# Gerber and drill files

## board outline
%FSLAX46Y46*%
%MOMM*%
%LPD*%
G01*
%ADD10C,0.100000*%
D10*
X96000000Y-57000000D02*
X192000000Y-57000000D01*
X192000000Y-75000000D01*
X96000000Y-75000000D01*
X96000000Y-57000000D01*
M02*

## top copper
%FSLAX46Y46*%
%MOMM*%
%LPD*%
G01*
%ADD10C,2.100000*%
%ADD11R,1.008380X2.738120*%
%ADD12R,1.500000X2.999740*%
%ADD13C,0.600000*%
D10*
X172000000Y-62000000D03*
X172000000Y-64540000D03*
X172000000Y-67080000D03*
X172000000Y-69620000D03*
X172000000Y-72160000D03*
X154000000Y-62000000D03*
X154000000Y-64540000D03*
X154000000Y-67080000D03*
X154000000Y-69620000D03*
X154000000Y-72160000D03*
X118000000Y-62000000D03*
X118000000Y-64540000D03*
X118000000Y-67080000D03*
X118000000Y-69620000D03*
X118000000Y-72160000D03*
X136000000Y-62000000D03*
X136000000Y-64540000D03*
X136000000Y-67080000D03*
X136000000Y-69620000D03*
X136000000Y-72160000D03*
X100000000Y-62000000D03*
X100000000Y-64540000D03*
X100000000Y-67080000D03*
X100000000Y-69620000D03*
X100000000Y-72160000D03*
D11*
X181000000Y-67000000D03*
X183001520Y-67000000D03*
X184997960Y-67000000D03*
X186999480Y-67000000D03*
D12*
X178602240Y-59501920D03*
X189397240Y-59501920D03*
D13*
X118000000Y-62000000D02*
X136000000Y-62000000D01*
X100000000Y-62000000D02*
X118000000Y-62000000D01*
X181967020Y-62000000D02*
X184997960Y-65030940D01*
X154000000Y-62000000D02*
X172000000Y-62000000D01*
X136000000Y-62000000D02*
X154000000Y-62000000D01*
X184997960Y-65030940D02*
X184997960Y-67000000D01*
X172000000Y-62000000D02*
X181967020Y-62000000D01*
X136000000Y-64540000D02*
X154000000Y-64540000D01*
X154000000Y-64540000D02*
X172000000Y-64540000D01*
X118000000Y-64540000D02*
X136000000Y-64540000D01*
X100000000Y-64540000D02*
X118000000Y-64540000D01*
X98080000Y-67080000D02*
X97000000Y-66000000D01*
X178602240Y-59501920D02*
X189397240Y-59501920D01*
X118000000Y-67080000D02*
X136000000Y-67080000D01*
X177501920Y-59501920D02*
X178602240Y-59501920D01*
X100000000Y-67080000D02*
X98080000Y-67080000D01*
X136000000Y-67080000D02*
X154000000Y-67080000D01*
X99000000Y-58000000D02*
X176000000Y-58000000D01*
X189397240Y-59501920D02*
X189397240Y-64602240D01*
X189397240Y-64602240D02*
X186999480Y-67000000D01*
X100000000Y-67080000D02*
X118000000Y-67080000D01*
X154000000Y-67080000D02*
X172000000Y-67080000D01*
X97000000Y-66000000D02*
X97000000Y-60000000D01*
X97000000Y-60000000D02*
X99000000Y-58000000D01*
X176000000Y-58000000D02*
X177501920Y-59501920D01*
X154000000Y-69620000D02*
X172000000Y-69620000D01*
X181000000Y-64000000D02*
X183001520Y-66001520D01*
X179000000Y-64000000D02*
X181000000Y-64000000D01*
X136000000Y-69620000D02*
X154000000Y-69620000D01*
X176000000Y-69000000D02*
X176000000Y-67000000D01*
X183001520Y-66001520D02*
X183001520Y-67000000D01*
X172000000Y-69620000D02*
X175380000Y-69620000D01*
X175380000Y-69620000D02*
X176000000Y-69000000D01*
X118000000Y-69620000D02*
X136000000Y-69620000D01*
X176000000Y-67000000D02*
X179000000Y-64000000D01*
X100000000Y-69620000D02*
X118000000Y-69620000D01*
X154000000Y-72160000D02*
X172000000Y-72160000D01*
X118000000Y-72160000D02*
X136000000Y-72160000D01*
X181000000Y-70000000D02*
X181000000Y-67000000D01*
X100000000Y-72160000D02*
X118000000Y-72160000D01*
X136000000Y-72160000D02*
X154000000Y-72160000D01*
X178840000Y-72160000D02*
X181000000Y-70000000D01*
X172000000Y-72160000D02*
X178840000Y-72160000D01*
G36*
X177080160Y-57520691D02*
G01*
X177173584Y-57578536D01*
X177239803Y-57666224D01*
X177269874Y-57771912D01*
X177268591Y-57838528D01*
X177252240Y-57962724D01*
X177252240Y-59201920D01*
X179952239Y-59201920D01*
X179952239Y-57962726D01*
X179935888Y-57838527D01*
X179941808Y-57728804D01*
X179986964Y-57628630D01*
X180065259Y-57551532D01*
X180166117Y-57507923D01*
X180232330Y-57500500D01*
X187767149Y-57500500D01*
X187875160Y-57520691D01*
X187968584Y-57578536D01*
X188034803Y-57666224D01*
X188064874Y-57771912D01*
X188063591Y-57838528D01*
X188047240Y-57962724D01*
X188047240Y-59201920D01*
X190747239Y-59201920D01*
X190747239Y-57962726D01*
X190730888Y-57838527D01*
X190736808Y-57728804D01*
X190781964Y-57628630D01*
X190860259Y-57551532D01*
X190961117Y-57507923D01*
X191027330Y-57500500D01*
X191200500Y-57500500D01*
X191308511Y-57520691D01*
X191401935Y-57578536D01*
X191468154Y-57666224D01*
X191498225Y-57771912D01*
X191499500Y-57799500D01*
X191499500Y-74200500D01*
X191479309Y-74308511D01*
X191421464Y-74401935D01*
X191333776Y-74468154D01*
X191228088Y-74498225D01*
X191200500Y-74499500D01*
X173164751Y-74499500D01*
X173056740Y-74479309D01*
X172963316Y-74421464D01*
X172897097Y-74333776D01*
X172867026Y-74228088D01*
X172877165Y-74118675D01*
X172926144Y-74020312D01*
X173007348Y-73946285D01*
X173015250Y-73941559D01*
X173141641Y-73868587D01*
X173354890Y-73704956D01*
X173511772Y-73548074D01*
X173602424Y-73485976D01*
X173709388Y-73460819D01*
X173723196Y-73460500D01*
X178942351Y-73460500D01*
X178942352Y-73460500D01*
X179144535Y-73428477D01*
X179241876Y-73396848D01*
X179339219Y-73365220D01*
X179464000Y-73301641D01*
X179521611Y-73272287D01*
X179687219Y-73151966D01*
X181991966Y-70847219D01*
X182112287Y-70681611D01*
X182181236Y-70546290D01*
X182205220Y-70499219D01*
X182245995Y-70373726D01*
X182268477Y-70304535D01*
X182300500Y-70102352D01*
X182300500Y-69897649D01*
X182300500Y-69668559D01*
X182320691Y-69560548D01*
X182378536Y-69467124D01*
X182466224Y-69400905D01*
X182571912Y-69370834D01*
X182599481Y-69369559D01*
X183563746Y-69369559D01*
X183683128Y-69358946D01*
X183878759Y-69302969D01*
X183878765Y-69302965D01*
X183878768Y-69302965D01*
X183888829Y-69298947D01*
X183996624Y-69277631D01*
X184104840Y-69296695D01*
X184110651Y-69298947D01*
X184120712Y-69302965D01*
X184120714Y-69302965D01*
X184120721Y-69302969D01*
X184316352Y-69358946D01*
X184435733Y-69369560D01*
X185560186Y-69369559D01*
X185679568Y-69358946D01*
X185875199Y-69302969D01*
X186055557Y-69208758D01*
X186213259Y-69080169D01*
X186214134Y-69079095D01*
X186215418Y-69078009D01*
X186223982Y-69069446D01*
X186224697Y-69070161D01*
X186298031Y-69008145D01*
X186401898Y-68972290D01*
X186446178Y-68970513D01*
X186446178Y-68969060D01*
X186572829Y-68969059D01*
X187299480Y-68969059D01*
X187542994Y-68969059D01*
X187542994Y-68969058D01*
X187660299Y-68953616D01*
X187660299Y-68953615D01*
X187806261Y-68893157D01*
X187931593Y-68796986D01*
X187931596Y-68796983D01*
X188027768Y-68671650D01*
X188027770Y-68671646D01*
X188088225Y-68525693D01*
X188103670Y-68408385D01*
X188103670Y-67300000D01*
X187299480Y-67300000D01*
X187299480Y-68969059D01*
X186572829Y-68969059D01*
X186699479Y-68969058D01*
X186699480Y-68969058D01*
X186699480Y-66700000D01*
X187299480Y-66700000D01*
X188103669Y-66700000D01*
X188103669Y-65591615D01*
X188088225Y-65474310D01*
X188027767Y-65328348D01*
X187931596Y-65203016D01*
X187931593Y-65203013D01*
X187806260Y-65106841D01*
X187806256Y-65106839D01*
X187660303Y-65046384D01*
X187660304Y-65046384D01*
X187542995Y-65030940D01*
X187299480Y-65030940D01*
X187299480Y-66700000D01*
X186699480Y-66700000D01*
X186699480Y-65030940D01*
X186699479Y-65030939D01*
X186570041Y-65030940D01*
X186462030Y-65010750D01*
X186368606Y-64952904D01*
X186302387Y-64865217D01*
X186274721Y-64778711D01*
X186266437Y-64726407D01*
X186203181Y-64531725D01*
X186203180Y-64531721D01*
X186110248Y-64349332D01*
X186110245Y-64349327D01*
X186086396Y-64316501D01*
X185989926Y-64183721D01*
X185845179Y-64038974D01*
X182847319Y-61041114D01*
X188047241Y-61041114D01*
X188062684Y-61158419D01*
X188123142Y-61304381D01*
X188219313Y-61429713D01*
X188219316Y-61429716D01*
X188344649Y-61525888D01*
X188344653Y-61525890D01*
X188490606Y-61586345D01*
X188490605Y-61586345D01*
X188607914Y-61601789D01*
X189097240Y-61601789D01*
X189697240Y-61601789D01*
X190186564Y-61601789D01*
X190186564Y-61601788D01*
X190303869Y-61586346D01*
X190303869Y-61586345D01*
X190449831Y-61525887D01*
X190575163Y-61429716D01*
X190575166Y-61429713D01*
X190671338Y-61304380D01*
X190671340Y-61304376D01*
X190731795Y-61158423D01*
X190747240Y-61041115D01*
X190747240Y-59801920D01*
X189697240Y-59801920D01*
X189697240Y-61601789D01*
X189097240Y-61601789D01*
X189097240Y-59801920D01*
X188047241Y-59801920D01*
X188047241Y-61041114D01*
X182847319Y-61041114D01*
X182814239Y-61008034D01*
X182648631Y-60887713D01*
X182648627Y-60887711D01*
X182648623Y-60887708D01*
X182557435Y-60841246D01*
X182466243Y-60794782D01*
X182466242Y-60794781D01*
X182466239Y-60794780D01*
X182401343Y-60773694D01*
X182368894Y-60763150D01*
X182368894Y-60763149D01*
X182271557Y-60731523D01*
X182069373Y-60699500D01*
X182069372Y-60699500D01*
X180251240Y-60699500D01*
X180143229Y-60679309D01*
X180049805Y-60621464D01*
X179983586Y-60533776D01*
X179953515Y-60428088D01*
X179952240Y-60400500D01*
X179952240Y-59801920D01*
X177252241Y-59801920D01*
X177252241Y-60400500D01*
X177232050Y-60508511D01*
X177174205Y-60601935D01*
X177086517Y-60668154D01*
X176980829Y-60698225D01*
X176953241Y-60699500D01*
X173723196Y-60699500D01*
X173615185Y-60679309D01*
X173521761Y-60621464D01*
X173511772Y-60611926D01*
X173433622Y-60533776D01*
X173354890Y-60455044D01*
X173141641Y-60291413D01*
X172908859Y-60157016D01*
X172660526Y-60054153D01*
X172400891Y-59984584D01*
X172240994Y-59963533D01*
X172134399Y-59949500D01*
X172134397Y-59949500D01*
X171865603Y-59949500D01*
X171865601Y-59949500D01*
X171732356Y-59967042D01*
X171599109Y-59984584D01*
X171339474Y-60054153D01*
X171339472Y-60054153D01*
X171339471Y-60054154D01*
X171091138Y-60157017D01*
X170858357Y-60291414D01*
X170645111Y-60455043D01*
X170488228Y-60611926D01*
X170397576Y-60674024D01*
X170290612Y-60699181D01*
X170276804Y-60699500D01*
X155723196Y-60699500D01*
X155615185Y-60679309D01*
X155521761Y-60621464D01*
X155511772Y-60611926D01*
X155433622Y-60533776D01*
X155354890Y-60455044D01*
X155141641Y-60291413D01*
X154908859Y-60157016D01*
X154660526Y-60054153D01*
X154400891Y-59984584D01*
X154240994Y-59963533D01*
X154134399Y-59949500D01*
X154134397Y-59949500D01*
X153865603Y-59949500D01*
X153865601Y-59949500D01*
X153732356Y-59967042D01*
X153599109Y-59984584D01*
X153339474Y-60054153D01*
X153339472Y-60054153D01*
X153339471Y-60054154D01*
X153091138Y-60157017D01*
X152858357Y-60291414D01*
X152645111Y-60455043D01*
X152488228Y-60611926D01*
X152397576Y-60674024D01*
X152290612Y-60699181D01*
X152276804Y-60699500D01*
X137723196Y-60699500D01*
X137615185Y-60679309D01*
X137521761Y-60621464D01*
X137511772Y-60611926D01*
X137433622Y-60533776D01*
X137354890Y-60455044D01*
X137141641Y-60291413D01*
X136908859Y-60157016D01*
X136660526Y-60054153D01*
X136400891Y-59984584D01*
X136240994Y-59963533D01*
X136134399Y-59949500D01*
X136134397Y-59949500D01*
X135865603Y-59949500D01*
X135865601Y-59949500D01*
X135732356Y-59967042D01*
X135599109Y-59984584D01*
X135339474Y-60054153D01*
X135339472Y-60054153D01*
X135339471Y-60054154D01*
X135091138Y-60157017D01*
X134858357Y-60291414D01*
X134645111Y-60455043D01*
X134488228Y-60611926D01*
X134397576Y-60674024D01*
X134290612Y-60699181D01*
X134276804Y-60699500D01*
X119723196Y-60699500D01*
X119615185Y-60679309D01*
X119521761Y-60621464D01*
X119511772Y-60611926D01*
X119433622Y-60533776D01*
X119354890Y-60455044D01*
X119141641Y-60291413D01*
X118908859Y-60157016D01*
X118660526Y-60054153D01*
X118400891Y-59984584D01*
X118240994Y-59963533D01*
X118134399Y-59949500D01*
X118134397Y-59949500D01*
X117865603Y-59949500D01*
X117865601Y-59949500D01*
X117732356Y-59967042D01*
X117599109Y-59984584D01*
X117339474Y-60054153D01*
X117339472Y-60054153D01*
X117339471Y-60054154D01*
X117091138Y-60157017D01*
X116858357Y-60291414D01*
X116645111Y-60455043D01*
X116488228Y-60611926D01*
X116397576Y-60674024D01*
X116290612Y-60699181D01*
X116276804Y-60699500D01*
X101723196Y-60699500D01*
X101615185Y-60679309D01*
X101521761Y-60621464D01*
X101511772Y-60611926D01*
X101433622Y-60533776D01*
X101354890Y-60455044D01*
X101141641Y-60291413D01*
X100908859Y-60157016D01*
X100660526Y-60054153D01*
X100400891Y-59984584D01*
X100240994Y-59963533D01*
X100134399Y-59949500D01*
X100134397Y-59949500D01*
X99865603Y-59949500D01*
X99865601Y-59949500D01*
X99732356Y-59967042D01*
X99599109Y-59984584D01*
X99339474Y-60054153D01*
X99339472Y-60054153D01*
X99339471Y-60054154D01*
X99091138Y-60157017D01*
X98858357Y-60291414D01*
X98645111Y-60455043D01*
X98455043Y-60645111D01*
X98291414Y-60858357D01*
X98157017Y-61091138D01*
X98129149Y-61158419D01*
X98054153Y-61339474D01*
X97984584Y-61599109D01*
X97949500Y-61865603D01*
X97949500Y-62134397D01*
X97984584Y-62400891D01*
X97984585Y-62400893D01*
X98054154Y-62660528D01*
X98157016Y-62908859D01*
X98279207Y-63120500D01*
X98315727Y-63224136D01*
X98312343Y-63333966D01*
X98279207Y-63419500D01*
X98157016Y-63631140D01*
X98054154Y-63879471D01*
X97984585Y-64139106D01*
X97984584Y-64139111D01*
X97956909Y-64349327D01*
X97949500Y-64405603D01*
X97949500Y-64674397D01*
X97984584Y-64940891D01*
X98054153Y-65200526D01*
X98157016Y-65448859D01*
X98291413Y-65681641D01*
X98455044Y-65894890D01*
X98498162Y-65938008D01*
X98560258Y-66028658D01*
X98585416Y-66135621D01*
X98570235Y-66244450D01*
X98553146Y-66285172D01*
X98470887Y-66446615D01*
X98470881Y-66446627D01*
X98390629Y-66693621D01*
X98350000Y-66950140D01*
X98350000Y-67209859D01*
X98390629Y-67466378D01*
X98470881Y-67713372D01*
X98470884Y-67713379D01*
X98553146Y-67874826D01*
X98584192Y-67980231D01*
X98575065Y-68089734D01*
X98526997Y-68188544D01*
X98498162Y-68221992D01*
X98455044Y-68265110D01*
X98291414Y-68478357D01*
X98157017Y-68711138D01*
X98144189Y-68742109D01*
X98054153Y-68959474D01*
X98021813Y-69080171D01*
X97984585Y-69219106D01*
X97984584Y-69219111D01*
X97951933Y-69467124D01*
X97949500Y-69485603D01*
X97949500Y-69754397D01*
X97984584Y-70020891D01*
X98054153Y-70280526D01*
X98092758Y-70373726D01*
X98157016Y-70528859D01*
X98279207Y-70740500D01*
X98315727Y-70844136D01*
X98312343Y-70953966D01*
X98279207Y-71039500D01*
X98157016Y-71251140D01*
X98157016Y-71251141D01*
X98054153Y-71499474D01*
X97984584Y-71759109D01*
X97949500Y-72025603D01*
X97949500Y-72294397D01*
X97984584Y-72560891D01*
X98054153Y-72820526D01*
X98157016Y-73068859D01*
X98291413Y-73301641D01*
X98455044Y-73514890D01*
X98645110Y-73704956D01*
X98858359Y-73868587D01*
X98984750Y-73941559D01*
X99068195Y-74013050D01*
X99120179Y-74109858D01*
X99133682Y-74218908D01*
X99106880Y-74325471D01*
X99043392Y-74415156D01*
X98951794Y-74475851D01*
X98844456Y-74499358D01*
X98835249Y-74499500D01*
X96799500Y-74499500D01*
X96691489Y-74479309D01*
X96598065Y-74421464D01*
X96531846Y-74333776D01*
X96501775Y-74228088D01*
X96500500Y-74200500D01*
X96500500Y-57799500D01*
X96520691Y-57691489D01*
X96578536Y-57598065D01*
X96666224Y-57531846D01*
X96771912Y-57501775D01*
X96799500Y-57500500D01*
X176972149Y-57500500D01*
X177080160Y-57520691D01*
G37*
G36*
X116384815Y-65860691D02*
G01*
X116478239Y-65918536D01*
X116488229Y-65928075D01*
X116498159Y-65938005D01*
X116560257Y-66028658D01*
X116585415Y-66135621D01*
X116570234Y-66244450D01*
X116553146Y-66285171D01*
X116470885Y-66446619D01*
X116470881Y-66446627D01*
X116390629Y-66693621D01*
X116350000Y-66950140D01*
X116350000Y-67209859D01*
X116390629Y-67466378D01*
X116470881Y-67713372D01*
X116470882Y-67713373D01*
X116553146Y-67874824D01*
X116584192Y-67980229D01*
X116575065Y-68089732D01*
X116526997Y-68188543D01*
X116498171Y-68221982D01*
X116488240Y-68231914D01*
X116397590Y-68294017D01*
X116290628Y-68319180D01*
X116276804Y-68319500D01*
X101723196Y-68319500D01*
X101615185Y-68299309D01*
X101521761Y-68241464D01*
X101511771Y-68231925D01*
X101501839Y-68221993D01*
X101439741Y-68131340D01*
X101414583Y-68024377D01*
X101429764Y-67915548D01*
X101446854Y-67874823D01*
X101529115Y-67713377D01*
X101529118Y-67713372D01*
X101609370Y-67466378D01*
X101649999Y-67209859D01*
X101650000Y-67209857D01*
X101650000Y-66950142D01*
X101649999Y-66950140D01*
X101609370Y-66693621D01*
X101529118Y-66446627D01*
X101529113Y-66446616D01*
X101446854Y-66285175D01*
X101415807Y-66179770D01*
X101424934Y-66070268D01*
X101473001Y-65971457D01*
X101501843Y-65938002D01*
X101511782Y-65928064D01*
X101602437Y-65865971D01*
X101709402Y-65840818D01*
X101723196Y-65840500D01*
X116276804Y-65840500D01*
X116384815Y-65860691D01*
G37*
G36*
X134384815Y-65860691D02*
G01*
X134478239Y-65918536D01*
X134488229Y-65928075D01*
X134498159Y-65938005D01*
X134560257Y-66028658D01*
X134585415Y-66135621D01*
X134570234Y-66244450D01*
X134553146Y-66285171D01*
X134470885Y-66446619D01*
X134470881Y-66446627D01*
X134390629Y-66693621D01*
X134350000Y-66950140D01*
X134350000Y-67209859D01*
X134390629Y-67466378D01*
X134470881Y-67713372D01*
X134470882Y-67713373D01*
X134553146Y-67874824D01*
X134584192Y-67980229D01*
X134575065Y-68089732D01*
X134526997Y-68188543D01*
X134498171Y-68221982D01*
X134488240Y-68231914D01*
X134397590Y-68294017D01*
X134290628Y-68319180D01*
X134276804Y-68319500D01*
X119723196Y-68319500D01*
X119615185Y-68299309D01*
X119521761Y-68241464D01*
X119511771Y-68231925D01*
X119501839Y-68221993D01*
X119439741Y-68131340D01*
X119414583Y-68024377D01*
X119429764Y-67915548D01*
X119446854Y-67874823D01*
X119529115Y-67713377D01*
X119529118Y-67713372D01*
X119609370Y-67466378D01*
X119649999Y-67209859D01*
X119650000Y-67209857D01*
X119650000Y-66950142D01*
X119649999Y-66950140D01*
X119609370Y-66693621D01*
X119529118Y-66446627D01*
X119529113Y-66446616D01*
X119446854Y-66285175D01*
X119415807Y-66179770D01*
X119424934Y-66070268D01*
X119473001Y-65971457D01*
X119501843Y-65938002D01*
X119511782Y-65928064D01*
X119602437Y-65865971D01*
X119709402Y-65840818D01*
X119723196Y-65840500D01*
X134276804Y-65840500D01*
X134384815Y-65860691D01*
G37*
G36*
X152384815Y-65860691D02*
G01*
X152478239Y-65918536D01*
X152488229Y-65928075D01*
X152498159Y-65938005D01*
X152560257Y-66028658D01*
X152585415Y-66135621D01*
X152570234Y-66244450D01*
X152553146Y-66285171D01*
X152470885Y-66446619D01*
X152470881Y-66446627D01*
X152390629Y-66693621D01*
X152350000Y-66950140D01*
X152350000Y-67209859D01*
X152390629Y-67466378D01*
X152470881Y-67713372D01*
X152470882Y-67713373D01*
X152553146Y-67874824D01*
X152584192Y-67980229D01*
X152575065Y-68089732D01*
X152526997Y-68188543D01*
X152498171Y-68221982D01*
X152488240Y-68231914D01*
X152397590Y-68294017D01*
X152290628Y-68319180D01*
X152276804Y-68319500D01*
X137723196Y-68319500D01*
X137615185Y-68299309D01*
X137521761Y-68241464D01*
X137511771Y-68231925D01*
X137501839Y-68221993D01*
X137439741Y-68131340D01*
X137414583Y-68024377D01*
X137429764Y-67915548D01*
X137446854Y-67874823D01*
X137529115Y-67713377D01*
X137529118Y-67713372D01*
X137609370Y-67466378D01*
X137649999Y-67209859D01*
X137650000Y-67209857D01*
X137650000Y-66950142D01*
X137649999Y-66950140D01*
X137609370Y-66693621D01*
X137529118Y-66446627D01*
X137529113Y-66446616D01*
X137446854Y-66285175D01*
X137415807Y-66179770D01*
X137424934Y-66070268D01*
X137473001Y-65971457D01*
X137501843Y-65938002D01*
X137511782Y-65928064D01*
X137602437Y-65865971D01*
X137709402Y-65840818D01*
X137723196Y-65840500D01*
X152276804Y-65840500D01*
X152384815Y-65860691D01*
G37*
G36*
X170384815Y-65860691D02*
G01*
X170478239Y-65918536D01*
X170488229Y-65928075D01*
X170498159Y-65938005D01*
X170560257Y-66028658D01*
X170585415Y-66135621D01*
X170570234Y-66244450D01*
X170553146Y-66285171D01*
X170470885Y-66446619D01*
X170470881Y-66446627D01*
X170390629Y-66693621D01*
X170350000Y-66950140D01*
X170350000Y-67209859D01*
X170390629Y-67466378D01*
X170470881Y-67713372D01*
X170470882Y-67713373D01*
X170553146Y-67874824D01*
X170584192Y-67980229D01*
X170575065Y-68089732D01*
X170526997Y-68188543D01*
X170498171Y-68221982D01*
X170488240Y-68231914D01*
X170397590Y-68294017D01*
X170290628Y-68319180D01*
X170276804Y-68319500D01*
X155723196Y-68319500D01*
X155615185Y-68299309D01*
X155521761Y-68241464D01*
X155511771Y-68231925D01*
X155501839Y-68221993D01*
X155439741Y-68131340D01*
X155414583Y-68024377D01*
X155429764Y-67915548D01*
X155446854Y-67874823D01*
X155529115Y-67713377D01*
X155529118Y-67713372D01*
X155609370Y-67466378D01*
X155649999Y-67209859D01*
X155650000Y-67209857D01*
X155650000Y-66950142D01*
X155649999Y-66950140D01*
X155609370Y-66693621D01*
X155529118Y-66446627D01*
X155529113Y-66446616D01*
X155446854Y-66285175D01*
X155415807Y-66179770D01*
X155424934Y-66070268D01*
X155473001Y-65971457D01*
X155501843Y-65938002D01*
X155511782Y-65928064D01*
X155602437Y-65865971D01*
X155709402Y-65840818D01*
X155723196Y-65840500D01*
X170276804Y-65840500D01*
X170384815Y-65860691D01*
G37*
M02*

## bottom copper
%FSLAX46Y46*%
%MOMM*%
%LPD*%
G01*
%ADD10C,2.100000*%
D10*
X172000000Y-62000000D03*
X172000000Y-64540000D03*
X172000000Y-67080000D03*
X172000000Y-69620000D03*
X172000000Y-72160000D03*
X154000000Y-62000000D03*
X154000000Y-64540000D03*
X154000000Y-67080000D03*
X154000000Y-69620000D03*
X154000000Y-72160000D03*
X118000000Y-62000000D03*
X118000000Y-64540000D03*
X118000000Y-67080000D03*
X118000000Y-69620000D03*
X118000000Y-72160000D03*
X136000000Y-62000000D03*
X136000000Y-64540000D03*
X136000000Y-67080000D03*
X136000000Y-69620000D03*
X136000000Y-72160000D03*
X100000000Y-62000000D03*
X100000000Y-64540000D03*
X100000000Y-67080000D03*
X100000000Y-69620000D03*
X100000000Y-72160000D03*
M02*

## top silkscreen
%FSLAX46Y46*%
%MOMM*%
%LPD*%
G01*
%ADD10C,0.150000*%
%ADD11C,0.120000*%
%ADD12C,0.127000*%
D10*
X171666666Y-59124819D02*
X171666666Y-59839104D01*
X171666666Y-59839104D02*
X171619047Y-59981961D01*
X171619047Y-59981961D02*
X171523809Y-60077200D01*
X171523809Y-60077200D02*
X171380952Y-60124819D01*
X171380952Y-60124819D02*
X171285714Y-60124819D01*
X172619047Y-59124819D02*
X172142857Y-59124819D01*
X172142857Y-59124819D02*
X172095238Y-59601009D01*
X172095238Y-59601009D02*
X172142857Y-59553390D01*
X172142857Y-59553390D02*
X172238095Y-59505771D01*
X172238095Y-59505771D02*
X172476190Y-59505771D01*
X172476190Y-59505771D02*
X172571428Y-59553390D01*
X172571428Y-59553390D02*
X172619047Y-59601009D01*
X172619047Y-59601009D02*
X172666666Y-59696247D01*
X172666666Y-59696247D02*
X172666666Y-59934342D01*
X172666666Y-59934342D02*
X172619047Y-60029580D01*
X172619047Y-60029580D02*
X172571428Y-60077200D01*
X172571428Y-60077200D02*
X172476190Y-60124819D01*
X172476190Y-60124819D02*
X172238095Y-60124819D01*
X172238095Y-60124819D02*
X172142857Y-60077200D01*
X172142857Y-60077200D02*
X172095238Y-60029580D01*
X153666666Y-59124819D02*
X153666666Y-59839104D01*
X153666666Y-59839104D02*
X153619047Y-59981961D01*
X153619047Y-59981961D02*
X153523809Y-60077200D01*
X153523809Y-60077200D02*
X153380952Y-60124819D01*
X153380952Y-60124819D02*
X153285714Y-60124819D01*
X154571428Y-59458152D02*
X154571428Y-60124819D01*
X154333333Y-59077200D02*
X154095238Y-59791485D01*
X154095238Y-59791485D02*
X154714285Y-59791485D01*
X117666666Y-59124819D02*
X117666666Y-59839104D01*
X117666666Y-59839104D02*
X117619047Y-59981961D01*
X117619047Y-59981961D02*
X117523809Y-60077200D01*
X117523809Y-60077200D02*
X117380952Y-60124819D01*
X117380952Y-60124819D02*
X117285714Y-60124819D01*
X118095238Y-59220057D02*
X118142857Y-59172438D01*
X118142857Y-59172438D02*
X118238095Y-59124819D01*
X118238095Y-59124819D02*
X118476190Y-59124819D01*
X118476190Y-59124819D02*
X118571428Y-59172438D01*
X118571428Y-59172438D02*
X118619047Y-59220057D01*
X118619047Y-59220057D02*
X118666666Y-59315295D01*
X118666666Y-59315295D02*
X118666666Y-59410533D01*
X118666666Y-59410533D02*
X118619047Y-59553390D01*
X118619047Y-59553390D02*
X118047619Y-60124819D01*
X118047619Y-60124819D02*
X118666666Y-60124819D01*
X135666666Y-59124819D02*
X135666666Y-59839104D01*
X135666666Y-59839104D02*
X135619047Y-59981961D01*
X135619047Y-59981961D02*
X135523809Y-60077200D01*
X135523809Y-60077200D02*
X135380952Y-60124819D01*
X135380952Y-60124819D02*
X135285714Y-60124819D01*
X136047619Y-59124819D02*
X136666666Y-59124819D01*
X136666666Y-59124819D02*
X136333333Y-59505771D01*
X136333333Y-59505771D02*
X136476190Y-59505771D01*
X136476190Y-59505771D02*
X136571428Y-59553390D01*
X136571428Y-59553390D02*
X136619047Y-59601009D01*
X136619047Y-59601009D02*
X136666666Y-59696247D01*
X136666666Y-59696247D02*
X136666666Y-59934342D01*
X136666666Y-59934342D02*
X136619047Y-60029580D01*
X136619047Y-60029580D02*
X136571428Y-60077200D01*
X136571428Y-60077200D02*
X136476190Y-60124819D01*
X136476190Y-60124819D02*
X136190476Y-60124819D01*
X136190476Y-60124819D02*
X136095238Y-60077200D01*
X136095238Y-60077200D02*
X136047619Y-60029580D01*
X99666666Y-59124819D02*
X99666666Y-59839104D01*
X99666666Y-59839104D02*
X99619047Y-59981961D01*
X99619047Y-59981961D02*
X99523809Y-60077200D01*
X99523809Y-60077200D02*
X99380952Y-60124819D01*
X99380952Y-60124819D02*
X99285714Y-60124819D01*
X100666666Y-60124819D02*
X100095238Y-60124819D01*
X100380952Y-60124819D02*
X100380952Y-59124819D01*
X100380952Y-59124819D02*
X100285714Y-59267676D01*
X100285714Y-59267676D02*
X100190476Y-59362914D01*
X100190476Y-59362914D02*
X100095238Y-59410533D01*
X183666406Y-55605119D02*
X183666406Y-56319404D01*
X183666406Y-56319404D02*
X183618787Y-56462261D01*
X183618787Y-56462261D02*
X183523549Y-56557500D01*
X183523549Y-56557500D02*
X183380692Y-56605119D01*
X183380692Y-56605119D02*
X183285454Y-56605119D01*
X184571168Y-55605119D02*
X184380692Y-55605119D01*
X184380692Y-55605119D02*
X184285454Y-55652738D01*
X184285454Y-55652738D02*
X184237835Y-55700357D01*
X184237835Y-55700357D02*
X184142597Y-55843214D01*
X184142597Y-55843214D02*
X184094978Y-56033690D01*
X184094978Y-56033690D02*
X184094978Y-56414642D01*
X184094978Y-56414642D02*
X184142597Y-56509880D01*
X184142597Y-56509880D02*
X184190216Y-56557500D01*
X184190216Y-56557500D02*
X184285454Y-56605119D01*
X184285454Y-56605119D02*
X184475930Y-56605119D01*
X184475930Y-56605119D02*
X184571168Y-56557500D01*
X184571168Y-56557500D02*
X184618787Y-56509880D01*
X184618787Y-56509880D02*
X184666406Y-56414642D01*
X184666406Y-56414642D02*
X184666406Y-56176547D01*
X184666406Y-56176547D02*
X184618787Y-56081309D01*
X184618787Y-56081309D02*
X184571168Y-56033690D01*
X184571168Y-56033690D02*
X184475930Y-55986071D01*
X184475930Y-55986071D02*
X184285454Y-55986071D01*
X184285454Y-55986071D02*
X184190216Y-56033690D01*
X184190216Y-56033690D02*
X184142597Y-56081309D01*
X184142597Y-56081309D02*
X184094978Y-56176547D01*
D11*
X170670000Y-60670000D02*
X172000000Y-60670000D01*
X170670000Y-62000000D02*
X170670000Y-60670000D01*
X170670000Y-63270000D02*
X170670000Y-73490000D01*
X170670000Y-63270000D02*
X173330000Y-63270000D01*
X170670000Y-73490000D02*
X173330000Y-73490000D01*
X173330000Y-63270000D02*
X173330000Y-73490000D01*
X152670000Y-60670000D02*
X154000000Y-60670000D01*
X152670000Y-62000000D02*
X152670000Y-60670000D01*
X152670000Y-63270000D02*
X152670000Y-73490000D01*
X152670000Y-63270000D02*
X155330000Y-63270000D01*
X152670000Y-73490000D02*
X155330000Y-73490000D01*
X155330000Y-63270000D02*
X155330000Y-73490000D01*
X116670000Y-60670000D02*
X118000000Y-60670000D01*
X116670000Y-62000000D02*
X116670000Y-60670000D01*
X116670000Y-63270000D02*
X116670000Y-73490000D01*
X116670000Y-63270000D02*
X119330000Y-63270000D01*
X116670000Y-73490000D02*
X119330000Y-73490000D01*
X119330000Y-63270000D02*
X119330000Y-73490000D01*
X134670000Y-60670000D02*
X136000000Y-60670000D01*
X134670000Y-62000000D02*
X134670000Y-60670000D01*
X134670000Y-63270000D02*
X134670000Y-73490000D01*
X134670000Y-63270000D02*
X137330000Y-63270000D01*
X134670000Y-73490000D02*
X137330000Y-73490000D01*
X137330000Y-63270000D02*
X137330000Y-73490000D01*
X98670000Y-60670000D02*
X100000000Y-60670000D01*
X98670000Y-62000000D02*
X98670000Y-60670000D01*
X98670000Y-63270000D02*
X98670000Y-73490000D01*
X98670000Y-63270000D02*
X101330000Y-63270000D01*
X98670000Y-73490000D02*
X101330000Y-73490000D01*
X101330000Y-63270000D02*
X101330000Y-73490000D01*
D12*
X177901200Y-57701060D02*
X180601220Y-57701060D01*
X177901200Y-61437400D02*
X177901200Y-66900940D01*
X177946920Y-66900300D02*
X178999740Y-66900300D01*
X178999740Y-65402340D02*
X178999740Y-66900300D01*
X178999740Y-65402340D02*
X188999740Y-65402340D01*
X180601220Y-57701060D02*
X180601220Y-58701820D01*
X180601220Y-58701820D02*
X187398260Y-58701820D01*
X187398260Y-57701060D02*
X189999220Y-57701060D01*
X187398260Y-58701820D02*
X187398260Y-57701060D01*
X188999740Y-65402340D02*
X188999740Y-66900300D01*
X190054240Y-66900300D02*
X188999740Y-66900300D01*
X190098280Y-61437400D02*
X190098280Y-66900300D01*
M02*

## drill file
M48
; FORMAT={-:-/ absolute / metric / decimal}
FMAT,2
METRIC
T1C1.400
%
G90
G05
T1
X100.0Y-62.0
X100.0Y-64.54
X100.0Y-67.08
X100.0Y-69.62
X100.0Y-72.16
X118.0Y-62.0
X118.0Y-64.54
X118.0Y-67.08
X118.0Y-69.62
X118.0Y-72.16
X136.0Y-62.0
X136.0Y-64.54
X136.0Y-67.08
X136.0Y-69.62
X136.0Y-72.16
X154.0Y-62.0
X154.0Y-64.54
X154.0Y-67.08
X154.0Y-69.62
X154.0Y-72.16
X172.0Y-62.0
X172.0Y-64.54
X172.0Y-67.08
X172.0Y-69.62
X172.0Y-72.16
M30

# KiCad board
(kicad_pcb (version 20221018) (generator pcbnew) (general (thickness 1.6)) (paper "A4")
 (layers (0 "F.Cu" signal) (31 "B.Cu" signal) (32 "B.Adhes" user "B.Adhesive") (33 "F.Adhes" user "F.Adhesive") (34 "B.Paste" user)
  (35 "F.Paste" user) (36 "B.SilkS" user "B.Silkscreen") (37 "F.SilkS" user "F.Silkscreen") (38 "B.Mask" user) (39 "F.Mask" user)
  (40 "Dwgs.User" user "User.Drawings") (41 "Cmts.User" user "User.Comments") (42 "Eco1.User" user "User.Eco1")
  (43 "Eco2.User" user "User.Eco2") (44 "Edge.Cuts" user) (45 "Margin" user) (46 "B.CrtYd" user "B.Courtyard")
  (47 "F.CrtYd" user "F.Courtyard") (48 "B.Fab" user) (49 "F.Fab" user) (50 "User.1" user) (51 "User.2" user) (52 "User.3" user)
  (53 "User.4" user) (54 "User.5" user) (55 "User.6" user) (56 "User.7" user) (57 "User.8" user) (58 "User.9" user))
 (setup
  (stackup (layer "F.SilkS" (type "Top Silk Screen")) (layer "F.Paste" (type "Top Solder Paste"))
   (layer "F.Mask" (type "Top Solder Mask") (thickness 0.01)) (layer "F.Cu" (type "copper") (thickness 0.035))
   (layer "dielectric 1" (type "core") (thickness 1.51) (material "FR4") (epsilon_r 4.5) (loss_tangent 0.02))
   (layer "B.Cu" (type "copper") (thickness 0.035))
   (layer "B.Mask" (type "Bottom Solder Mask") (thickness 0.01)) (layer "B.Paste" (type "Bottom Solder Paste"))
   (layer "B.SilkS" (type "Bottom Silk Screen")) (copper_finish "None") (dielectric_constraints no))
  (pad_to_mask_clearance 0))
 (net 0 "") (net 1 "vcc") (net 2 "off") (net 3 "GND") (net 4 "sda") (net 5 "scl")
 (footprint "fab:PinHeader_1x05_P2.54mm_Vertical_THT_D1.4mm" (layer "F.Cu") (at 172 62)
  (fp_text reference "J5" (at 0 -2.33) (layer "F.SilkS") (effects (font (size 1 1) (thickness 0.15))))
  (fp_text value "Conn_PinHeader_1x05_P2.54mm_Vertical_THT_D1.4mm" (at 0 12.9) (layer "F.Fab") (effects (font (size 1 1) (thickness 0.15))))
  (fp_line (start -1.33 -1.33) (end 0 -1.33) (stroke (width 0.12) (type solid)) (layer "F.SilkS"))
  (fp_line (start -1.33 0) (end -1.33 -1.33) (stroke (width 0.12) (type solid)) (layer "F.SilkS"))
  (fp_line (start -1.33 1.27) (end -1.33 11.49) (stroke (width 0.12) (type solid)) (layer "F.SilkS"))
  (fp_line (start -1.33 1.27) (end 1.33 1.27) (stroke (width 0.12) (type solid)) (layer "F.SilkS"))
  (fp_line (start -1.33 11.49) (end 1.33 11.49) (stroke (width 0.12) (type solid)) (layer "F.SilkS"))
  (fp_line (start 1.33 1.27) (end 1.33 11.49) (stroke (width 0.12) (type solid)) (layer "F.SilkS"))
  (pad "1" thru_hole circle (at 0 0) (size 2.1 2.1) (drill 1.4) (layers "*.Cu" "*.Mask") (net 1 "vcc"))
  (pad "2" thru_hole circle (at 0 2.54) (size 2.1 2.1) (drill 1.4) (layers "*.Cu" "*.Mask") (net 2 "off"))
  (pad "3" thru_hole circle (at 0 5.08) (size 2.1 2.1) (drill 1.4) (layers "*.Cu" "*.Mask") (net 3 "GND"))
  (pad "4" thru_hole circle (at 0 7.62) (size 2.1 2.1) (drill 1.4) (layers "*.Cu" "*.Mask") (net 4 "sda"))
  (pad "5" thru_hole circle (at 0 10.16) (size 2.1 2.1) (drill 1.4) (layers "*.Cu" "*.Mask") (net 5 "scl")))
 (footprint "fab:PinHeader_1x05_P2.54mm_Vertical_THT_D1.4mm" (layer "F.Cu") (at 154 62)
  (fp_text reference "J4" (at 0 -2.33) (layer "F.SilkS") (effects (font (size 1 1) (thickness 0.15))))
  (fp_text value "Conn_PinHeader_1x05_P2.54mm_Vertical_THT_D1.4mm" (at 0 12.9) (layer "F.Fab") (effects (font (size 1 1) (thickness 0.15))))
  (fp_line (start -1.33 -1.33) (end 0 -1.33) (stroke (width 0.12) (type solid)) (layer "F.SilkS"))
  (fp_line (start -1.33 0) (end -1.33 -1.33) (stroke (width 0.12) (type solid)) (layer "F.SilkS"))
  (fp_line (start -1.33 1.27) (end -1.33 11.49) (stroke (width 0.12) (type solid)) (layer "F.SilkS"))
  (fp_line (start -1.33 1.27) (end 1.33 1.27) (stroke (width 0.12) (type solid)) (layer "F.SilkS"))
  (fp_line (start -1.33 11.49) (end 1.33 11.49) (stroke (width 0.12) (type solid)) (layer "F.SilkS"))
  (fp_line (start 1.33 1.27) (end 1.33 11.49) (stroke (width 0.12) (type solid)) (layer "F.SilkS"))
  (pad "1" thru_hole circle (at 0 0) (size 2.1 2.1) (drill 1.4) (layers "*.Cu" "*.Mask") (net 1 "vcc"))
  (pad "2" thru_hole circle (at 0 2.54) (size 2.1 2.1) (drill 1.4) (layers "*.Cu" "*.Mask") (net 2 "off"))
  (pad "3" thru_hole circle (at 0 5.08) (size 2.1 2.1) (drill 1.4) (layers "*.Cu" "*.Mask") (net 3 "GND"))
  (pad "4" thru_hole circle (at 0 7.62) (size 2.1 2.1) (drill 1.4) (layers "*.Cu" "*.Mask") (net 4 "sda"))
  (pad "5" thru_hole circle (at 0 10.16) (size 2.1 2.1) (drill 1.4) (layers "*.Cu" "*.Mask") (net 5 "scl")))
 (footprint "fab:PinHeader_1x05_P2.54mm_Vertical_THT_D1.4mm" (layer "F.Cu") (at 118 62)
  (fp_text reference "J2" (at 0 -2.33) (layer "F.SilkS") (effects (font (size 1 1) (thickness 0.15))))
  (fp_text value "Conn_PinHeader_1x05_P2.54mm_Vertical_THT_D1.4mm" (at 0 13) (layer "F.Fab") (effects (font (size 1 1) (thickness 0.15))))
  (fp_line (start -1.33 -1.33) (end 0 -1.33) (stroke (width 0.12) (type solid)) (layer "F.SilkS"))
  (fp_line (start -1.33 0) (end -1.33 -1.33) (stroke (width 0.12) (type solid)) (layer "F.SilkS"))
  (fp_line (start -1.33 1.27) (end -1.33 11.49) (stroke (width 0.12) (type solid)) (layer "F.SilkS"))
  (fp_line (start -1.33 1.27) (end 1.33 1.27) (stroke (width 0.12) (type solid)) (layer "F.SilkS"))
  (fp_line (start -1.33 11.49) (end 1.33 11.49) (stroke (width 0.12) (type solid)) (layer "F.SilkS"))
  (fp_line (start 1.33 1.27) (end 1.33 11.49) (stroke (width 0.12) (type solid)) (layer "F.SilkS"))
  (pad "1" thru_hole circle (at 0 0) (size 2.1 2.1) (drill 1.4) (layers "*.Cu" "*.Mask") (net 1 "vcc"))
  (pad "2" thru_hole circle (at 0 2.54) (size 2.1 2.1) (drill 1.4) (layers "*.Cu" "*.Mask") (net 2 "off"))
  (pad "3" thru_hole circle (at 0 5.08) (size 2.1 2.1) (drill 1.4) (layers "*.Cu" "*.Mask") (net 3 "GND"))
  (pad "4" thru_hole circle (at 0 7.62) (size 2.1 2.1) (drill 1.4) (layers "*.Cu" "*.Mask") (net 4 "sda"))
  (pad "5" thru_hole circle (at 0 10.16) (size 2.1 2.1) (drill 1.4) (layers "*.Cu" "*.Mask") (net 5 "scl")))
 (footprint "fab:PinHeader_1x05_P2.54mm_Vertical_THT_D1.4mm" (layer "F.Cu") (at 136 62)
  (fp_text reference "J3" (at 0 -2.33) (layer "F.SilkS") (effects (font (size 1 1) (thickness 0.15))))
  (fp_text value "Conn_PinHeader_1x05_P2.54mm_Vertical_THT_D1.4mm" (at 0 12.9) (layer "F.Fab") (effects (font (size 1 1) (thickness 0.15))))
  (fp_line (start -1.33 -1.33) (end 0 -1.33) (stroke (width 0.12) (type solid)) (layer "F.SilkS"))
  (fp_line (start -1.33 0) (end -1.33 -1.33) (stroke (width 0.12) (type solid)) (layer "F.SilkS"))
  (fp_line (start -1.33 1.27) (end -1.33 11.49) (stroke (width 0.12) (type solid)) (layer "F.SilkS"))
  (fp_line (start -1.33 1.27) (end 1.33 1.27) (stroke (width 0.12) (type solid)) (layer "F.SilkS"))
  (fp_line (start -1.33 11.49) (end 1.33 11.49) (stroke (width 0.12) (type solid)) (layer "F.SilkS"))
  (fp_line (start 1.33 1.27) (end 1.33 11.49) (stroke (width 0.12) (type solid)) (layer "F.SilkS"))
  (pad "1" thru_hole circle (at 0 0) (size 2.1 2.1) (drill 1.4) (layers "*.Cu" "*.Mask") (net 1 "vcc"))
  (pad "2" thru_hole circle (at 0 2.54) (size 2.1 2.1) (drill 1.4) (layers "*.Cu" "*.Mask") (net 2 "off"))
  (pad "3" thru_hole circle (at 0 5.08) (size 2.1 2.1) (drill 1.4) (layers "*.Cu" "*.Mask") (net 3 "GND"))
  (pad "4" thru_hole circle (at 0 7.62) (size 2.1 2.1) (drill 1.4) (layers "*.Cu" "*.Mask") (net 4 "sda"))
  (pad "5" thru_hole circle (at 0 10.16) (size 2.1 2.1) (drill 1.4) (layers "*.Cu" "*.Mask") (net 5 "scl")))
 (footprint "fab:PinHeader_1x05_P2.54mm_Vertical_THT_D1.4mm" (layer "F.Cu") (at 100 62)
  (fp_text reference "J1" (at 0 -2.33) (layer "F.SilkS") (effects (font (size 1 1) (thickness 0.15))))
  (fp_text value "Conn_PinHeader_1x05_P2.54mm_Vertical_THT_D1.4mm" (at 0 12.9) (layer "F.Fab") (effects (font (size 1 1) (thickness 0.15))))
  (fp_line (start -1.33 -1.33) (end 0 -1.33) (stroke (width 0.12) (type solid)) (layer "F.SilkS"))
  (fp_line (start -1.33 0) (end -1.33 -1.33) (stroke (width 0.12) (type solid)) (layer "F.SilkS"))
  (fp_line (start -1.33 1.27) (end -1.33 11.49) (stroke (width 0.12) (type solid)) (layer "F.SilkS"))
  (fp_line (start -1.33 1.27) (end 1.33 1.27) (stroke (width 0.12) (type solid)) (layer "F.SilkS"))
  (fp_line (start -1.33 11.49) (end 1.33 11.49) (stroke (width 0.12) (type solid)) (layer "F.SilkS"))
  (fp_line (start 1.33 1.27) (end 1.33 11.49) (stroke (width 0.12) (type solid)) (layer "F.SilkS"))
  (pad "1" thru_hole circle (at 0 0) (size 2.1 2.1) (drill 1.4) (layers "*.Cu" "*.Mask") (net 1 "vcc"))
  (pad "2" thru_hole circle (at 0 2.54) (size 2.1 2.1) (drill 1.4) (layers "*.Cu" "*.Mask") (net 2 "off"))
  (pad "3" thru_hole circle (at 0 5.08) (size 2.1 2.1) (drill 1.4) (layers "*.Cu" "*.Mask") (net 3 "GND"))
  (pad "4" thru_hole circle (at 0 7.62) (size 2.1 2.1) (drill 1.4) (layers "*.Cu" "*.Mask") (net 4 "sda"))
  (pad "5" thru_hole circle (at 0 10.16) (size 2.1 2.1) (drill 1.4) (layers "*.Cu" "*.Mask") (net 5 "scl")))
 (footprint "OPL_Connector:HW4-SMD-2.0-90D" (layer "F.Cu") (at 183.99974 62.2003)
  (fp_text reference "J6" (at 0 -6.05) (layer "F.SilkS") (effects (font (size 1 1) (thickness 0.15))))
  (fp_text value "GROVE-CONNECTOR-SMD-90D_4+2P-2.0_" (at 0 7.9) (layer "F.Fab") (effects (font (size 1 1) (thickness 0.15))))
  (fp_line (start -6.09854 -4.49924) (end -3.39852 -4.49924) (stroke (width 0.127) (type solid)) (layer "F.SilkS"))
  (fp_line (start -6.09854 -0.7629) (end -6.09854 4.70064) (stroke (width 0.127) (type solid)) (layer "F.SilkS"))
  (fp_line (start -6.05282 4.7) (end -5 4.7) (stroke (width 0.127) (type solid)) (layer "F.SilkS"))
  (fp_line (start -5 3.20204) (end -5 4.7) (stroke (width 0.127) (type solid)) (layer "F.SilkS"))
  (fp_line (start -5 3.20204) (end 5 3.20204) (stroke (width 0.127) (type solid)) (layer "F.SilkS"))
  (fp_line (start -3.39852 -4.49924) (end -3.39852 -3.49848) (stroke (width 0.127) (type solid)) (layer "F.SilkS"))
  (fp_line (start -3.39852 -3.49848) (end 3.39852 -3.49848) (stroke (width 0.127) (type solid)) (layer "F.SilkS"))
  (fp_line (start 3.39852 -4.49924) (end 5.99948 -4.49924) (stroke (width 0.127) (type solid)) (layer "F.SilkS"))
  (fp_line (start 3.39852 -3.49848) (end 3.39852 -4.49924) (stroke (width 0.127) (type solid)) (layer "F.SilkS"))
  (fp_line (start 5 3.20204) (end 5 4.7) (stroke (width 0.127) (type solid)) (layer "F.SilkS"))
  (fp_line (start 6.0545 4.7) (end 5 4.7) (stroke (width 0.127) (type solid)) (layer "F.SilkS"))
  (fp_line (start 6.09854 -0.7629) (end 6.09854 4.7) (stroke (width 0.127) (type solid)) (layer "F.SilkS"))
  (pad "1" smd rect (at -2.99974 4.7997 90) (size 2.73812 1.00838) (layers "F.Cu" "F.Paste" "F.Mask") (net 5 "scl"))
  (pad "2" smd rect (at -0.99822 4.7997 90) (size 2.73812 1.00838) (layers "F.Cu" "F.Paste" "F.Mask") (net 4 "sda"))
  (pad "3" smd rect (at 0.99822 4.7997 90) (size 2.73812 1.00838) (layers "F.Cu" "F.Paste" "F.Mask") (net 1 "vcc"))
  (pad "4" smd rect (at 2.99974 4.7997 90) (size 2.73812 1.00838) (layers "F.Cu" "F.Paste" "F.Mask") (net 3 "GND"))
  (pad "5" smd rect (at -5.3975 -2.69838 90) (size 2.99974 1.5) (layers "F.Cu" "F.Paste" "F.Mask") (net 3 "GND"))
  (pad "6" smd rect (at 5.3975 -2.69838 90) (size 2.99974 1.5) (layers "F.Cu" "F.Paste" "F.Mask") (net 3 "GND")))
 (gr_rect (start 96 57) (end 192 75) (stroke (width 0.1) (type default)) (fill none) (layer "Edge.Cuts"))
 (segment (start 118 62) (end 136 62) (width 0.6) (layer "F.Cu") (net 1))
 (segment (start 100 62) (end 118 62) (width 0.6) (layer "F.Cu") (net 1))
 (segment (start 181.96702 62) (end 184.99796 65.03094) (width 0.6) (layer "F.Cu") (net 1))
 (segment (start 154 62) (end 172 62) (width 0.6) (layer "F.Cu") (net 1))
 (segment (start 136 62) (end 154 62) (width 0.6) (layer "F.Cu") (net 1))
 (segment (start 184.99796 65.03094) (end 184.99796 67) (width 0.6) (layer "F.Cu") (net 1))
 (segment (start 172 62) (end 181.96702 62) (width 0.6) (layer "F.Cu") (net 1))
 (segment (start 136 64.54) (end 154 64.54) (width 0.6) (layer "F.Cu") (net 2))
 (segment (start 154 64.54) (end 172 64.54) (width 0.6) (layer "F.Cu") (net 2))
 (segment (start 118 64.54) (end 136 64.54) (width 0.6) (layer "F.Cu") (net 2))
 (segment (start 100 64.54) (end 118 64.54) (width 0.6) (layer "F.Cu") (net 2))
 (segment (start 98.08 67.08) (end 97 66) (width 0.6) (layer "F.Cu") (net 3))
 (segment (start 178.60224 59.50192) (end 189.39724 59.50192) (width 0.6) (layer "F.Cu") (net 3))
 (segment (start 118 67.08) (end 136 67.08) (width 0.6) (layer "F.Cu") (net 3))
 (segment (start 177.50192 59.50192) (end 178.60224 59.50192) (width 0.6) (layer "F.Cu") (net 3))
 (segment (start 100 67.08) (end 98.08 67.08) (width 0.6) (layer "F.Cu") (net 3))
 (segment (start 136 67.08) (end 154 67.08) (width 0.6) (layer "F.Cu") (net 3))
 (segment (start 99 58) (end 176 58) (width 0.6) (layer "F.Cu") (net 3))
 (segment (start 189.39724 59.50192) (end 189.39724 64.60224) (width 0.6) (layer "F.Cu") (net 3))
 (segment (start 189.39724 64.60224) (end 186.99948 67) (width 0.6) (layer "F.Cu") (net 3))
 (segment (start 100 67.08) (end 118 67.08) (width 0.6) (layer "F.Cu") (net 3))
 (segment (start 154 67.08) (end 172 67.08) (width 0.6) (layer "F.Cu") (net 3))
 (segment (start 97 66) (end 97 60) (width 0.6) (layer "F.Cu") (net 3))
 (segment (start 97 60) (end 99 58) (width 0.6) (layer "F.Cu") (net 3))
 (segment (start 176 58) (end 177.50192 59.50192) (width 0.6) (layer "F.Cu") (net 3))
 (segment (start 154 69.62) (end 172 69.62) (width 0.6) (layer "F.Cu") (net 4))
 (segment (start 181 64) (end 183.00152 66.00152) (width 0.6) (layer "F.Cu") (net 4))
 (segment (start 179 64) (end 181 64) (width 0.6) (layer "F.Cu") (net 4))
 (segment (start 136 69.62) (end 154 69.62) (width 0.6) (layer "F.Cu") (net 4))
 (segment (start 176 69) (end 176 67) (width 0.6) (layer "F.Cu") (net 4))
 (segment (start 183.00152 66.00152) (end 183.00152 67) (width 0.6) (layer "F.Cu") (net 4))
 (segment (start 172 69.62) (end 175.38 69.62) (width 0.6) (layer "F.Cu") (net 4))
 (segment (start 175.38 69.62) (end 176 69) (width 0.6) (layer "F.Cu") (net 4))
 (segment (start 118 69.62) (end 136 69.62) (width 0.6) (layer "F.Cu") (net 4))
 (segment (start 176 67) (end 179 64) (width 0.6) (layer "F.Cu") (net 4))
 (segment (start 100 69.62) (end 118 69.62) (width 0.6) (layer "F.Cu") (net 4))
 (segment (start 154 72.16) (end 172 72.16) (width 0.6) (layer "F.Cu") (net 5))
 (segment (start 118 72.16) (end 136 72.16) (width 0.6) (layer "F.Cu") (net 5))
 (segment (start 181 70) (end 181 67) (width 0.6) (layer "F.Cu") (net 5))
 (segment (start 100 72.16) (end 118 72.16) (width 0.6) (layer "F.Cu") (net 5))
 (segment (start 136 72.16) (end 154 72.16) (width 0.6) (layer "F.Cu") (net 5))
 (segment (start 178.84 72.16) (end 181 70) (width 0.6) (layer "F.Cu") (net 5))
 (segment (start 172 72.16) (end 178.84 72.16) (width 0.6) (layer "F.Cu") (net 5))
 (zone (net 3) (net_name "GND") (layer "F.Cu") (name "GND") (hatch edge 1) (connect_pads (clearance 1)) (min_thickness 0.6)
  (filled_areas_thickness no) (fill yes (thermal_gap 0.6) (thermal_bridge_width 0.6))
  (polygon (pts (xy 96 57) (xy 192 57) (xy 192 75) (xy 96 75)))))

